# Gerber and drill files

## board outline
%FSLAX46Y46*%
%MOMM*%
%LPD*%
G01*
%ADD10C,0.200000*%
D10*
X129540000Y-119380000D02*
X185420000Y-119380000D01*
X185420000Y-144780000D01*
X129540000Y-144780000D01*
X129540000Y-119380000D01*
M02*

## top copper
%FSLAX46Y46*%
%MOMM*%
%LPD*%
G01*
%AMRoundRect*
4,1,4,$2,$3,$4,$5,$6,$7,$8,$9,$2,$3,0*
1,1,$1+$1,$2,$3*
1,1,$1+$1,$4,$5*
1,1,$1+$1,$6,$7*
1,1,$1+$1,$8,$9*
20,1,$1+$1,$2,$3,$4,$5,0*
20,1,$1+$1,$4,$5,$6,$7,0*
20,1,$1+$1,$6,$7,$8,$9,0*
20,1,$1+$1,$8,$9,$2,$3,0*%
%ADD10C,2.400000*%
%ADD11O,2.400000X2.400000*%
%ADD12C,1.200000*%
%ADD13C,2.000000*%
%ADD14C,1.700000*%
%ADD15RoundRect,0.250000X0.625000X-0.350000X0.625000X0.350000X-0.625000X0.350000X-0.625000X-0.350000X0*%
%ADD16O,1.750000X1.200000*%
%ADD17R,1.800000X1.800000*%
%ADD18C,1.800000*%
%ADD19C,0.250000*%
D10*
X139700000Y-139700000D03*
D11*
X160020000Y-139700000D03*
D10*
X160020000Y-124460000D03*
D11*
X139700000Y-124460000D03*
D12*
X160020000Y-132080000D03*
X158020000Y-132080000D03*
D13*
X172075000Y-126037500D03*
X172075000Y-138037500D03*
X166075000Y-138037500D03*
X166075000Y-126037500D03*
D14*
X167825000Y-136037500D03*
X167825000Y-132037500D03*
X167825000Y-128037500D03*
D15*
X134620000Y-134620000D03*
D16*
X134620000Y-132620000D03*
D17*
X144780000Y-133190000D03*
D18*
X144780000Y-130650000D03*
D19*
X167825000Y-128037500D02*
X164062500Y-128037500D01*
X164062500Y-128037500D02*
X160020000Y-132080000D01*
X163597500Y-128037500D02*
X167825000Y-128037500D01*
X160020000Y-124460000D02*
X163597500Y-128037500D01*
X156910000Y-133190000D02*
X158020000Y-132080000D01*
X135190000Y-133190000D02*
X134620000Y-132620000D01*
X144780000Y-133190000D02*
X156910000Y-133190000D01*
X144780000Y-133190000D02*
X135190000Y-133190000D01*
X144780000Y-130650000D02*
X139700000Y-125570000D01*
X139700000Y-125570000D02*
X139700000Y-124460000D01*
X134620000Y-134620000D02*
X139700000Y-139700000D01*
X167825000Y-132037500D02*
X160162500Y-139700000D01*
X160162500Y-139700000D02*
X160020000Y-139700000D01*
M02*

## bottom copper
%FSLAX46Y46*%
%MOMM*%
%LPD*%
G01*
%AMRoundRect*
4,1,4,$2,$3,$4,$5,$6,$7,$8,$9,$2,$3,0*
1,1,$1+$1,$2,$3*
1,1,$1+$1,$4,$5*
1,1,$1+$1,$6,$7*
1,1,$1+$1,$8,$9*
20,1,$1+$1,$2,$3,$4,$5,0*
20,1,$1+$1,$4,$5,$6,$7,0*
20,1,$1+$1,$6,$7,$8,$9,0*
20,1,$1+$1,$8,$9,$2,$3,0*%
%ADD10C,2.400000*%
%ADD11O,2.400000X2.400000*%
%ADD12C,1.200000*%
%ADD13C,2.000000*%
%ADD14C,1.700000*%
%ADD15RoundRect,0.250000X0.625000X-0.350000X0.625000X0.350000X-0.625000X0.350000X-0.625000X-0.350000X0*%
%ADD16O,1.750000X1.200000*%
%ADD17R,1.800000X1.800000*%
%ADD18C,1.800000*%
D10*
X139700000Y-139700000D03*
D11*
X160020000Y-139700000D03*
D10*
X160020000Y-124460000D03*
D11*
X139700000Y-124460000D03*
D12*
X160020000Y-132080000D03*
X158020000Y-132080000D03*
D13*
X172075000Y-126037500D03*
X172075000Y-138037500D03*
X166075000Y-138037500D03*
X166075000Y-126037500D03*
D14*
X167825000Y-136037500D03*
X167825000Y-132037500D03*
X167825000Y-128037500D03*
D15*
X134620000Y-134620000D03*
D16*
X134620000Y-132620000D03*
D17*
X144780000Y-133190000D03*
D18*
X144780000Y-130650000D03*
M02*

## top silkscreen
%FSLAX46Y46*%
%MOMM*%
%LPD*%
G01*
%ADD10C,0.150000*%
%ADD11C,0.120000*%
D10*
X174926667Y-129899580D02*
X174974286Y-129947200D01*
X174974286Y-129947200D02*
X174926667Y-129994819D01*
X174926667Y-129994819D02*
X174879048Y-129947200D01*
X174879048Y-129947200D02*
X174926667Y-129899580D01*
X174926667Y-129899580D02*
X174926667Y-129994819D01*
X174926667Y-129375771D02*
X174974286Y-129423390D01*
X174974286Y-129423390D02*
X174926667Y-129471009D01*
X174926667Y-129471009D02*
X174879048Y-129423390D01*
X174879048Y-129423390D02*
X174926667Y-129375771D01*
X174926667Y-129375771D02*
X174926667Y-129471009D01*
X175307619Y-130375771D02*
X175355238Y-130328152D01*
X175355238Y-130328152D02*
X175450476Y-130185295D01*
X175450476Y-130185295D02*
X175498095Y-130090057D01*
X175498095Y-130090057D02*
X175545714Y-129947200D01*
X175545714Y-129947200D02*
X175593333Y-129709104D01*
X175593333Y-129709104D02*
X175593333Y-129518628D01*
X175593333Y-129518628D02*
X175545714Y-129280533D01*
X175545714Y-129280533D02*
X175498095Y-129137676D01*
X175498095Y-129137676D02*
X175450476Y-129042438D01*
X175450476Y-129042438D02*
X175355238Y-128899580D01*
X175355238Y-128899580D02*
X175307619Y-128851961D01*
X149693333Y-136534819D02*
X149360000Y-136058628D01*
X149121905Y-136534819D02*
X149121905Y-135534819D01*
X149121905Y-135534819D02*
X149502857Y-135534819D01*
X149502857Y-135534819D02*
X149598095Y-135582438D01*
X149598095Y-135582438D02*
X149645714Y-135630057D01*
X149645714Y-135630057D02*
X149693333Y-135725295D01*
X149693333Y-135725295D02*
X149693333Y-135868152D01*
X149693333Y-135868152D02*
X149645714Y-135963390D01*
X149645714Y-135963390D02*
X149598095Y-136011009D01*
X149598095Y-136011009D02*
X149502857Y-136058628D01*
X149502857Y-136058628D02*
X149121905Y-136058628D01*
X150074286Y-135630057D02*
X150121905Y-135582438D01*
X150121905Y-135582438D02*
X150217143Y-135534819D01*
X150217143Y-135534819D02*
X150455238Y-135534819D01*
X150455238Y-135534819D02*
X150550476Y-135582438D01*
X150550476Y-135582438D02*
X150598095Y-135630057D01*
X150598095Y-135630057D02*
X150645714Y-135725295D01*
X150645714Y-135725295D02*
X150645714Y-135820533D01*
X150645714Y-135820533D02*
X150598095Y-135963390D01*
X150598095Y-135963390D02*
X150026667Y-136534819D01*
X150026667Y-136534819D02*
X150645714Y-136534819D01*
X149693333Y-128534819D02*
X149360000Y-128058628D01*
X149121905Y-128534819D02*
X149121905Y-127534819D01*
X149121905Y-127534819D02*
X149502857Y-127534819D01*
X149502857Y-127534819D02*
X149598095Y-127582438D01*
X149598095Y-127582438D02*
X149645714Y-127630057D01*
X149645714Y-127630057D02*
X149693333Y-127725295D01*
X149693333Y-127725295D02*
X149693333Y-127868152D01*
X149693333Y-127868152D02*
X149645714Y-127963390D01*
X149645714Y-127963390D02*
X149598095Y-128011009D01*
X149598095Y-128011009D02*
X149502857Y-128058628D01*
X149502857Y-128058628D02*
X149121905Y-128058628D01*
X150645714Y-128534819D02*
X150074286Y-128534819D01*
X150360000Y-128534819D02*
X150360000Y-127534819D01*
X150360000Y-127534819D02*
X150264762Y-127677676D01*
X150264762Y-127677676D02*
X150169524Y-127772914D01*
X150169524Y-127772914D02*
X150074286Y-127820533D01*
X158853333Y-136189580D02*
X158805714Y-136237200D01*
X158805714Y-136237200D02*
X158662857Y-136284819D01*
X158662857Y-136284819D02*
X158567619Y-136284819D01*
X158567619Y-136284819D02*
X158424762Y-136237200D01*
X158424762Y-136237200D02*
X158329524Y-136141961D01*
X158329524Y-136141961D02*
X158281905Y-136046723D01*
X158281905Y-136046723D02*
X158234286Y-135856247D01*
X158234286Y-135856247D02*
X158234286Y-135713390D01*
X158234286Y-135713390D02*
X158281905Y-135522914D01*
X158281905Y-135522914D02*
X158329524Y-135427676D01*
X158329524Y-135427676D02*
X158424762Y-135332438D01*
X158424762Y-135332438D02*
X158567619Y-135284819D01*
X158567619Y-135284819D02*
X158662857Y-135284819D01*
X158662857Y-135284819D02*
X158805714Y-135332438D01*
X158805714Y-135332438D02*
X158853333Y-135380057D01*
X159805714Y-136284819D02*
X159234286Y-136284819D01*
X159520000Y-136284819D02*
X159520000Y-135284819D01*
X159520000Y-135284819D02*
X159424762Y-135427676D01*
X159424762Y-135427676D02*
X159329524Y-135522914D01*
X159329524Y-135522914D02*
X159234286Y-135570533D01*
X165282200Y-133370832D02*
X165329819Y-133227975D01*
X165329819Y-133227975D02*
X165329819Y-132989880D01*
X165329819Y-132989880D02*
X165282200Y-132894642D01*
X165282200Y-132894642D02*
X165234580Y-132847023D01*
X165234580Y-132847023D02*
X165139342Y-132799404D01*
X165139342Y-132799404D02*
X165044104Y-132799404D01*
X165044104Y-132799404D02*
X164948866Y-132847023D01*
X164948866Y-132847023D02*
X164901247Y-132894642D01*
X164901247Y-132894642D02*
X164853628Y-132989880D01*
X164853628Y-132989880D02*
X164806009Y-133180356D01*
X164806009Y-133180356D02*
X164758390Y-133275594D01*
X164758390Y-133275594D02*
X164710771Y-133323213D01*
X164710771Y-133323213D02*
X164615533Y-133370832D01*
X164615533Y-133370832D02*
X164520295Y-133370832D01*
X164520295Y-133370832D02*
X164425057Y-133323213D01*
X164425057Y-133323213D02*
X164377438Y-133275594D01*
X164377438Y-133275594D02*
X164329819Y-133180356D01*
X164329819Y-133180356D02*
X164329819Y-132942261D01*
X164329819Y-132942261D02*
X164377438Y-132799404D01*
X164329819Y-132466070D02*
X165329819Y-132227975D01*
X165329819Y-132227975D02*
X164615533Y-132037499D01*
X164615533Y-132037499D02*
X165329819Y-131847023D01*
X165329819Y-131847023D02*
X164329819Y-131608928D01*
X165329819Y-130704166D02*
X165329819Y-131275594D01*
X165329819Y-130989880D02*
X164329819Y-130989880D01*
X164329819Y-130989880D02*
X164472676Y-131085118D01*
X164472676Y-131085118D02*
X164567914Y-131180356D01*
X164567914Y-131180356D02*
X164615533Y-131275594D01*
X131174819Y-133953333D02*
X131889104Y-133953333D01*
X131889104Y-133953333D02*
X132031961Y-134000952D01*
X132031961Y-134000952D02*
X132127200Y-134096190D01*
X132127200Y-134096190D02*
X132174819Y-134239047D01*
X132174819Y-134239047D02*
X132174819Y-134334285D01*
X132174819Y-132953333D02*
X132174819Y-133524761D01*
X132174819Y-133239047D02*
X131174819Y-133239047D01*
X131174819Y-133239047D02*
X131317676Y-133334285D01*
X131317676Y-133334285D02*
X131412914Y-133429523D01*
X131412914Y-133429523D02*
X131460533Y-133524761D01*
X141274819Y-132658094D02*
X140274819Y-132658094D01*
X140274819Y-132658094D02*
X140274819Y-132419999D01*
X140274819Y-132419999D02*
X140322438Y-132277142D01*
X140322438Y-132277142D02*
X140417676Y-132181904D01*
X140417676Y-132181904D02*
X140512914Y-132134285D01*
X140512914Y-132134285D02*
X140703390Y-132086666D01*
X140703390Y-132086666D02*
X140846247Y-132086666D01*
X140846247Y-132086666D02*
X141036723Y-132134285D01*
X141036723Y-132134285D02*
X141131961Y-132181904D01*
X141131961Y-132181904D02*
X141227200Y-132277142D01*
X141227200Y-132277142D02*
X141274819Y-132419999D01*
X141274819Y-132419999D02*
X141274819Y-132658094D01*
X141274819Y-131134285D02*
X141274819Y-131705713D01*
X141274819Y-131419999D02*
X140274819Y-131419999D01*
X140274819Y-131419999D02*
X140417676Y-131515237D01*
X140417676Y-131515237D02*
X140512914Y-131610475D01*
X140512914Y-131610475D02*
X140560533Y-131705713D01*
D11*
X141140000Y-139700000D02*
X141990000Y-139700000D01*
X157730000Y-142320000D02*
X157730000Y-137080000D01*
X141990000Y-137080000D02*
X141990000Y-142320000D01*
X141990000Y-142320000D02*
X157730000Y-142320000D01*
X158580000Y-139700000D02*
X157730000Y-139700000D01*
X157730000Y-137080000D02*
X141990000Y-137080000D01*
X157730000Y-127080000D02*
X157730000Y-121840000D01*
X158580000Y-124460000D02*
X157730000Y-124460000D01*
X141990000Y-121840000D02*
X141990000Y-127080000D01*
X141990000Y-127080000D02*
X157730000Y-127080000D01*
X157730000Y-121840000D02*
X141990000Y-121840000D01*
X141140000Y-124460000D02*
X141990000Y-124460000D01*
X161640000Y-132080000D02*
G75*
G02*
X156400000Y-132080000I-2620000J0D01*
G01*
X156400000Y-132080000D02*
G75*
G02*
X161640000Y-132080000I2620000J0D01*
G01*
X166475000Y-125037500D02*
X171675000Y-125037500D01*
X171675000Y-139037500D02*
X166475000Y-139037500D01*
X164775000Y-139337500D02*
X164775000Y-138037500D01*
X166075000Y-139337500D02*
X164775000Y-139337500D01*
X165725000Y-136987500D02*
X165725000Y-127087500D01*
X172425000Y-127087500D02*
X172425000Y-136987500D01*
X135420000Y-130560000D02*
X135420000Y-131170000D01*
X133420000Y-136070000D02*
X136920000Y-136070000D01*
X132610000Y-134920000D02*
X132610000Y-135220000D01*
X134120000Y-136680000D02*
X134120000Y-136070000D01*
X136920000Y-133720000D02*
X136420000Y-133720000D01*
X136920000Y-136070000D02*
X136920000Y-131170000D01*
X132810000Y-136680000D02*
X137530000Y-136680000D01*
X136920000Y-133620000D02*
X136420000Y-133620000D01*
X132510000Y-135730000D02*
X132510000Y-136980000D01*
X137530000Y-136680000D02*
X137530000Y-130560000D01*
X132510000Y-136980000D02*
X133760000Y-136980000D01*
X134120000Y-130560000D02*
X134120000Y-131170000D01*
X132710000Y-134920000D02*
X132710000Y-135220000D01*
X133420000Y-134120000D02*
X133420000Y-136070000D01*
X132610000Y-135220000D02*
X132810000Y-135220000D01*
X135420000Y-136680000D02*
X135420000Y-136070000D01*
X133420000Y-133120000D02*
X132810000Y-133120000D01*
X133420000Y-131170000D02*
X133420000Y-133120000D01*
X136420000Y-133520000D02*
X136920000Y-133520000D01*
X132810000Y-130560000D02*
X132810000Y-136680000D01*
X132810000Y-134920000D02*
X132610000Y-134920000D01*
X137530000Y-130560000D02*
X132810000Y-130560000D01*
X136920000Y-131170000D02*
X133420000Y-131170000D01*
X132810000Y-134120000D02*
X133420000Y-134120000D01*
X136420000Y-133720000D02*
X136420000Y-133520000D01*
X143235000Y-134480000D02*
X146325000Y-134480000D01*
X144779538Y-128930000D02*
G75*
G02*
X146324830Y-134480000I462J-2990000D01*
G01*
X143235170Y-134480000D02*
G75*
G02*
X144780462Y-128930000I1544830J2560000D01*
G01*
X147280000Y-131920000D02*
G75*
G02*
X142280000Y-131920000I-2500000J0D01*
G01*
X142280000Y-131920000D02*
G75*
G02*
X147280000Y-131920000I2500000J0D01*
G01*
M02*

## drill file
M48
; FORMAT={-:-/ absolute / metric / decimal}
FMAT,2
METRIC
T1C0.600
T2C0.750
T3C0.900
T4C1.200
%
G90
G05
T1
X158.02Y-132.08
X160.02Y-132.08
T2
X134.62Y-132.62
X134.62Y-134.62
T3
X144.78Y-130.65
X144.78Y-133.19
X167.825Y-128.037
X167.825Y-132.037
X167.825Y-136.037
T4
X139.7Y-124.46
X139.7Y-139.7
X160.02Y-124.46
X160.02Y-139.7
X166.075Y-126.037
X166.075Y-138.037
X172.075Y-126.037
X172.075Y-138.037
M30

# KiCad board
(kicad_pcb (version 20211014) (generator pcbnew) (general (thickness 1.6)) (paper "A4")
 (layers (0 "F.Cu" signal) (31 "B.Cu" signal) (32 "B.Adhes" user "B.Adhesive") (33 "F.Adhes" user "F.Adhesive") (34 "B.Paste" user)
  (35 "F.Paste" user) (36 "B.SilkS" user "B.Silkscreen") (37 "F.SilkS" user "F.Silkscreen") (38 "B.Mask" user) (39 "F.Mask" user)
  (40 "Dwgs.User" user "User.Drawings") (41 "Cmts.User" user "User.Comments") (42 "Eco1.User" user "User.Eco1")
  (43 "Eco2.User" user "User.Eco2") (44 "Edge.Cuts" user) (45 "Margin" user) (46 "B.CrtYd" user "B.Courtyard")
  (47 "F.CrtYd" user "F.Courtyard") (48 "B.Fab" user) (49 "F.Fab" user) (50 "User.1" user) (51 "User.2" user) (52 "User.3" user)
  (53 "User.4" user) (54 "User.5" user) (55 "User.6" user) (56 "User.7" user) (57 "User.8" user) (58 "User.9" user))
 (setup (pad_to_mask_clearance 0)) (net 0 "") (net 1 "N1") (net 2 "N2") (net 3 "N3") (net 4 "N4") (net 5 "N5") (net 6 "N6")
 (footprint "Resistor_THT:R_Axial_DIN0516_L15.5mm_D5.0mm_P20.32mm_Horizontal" (layer "F.Cu") (at 139.7 139.7)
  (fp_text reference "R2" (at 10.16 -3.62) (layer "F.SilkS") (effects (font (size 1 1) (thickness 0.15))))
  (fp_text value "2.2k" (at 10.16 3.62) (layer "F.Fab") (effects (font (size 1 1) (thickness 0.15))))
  (fp_line (start 1.44 0) (end 2.29 0) (layer "F.SilkS") (width 0.12))
  (fp_line (start 18.03 2.62) (end 18.03 -2.62) (layer "F.SilkS") (width 0.12))
  (fp_line (start 2.29 -2.62) (end 2.29 2.62) (layer "F.SilkS") (width 0.12))
  (fp_line (start 2.29 2.62) (end 18.03 2.62) (layer "F.SilkS") (width 0.12))
  (fp_line (start 18.88 0) (end 18.03 0) (layer "F.SilkS") (width 0.12))
  (fp_line (start 18.03 -2.62) (end 2.29 -2.62) (layer "F.SilkS") (width 0.12))
  (pad "1" thru_hole circle (at 0 0) (size 2.4 2.4) (drill 1.2) (layers *.Cu *.Mask) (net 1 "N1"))
  (pad "2" thru_hole oval (at 20.32 0) (size 2.4 2.4) (drill 1.2) (layers *.Cu *.Mask) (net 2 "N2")))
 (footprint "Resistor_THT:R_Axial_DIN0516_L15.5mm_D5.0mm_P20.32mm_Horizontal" (layer "F.Cu") (at 160.02 124.46 180)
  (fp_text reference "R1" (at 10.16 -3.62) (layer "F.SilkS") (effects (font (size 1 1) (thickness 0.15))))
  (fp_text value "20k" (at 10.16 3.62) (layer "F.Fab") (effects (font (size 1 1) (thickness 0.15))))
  (fp_line (start 2.29 -2.62) (end 2.29 2.62) (layer "F.SilkS") (width 0.12))
  (fp_line (start 1.44 0) (end 2.29 0) (layer "F.SilkS") (width 0.12))
  (fp_line (start 18.03 2.62) (end 18.03 -2.62) (layer "F.SilkS") (width 0.12))
  (fp_line (start 18.03 -2.62) (end 2.29 -2.62) (layer "F.SilkS") (width 0.12))
  (fp_line (start 2.29 2.62) (end 18.03 2.62) (layer "F.SilkS") (width 0.12))
  (fp_line (start 18.88 0) (end 18.03 0) (layer "F.SilkS") (width 0.12))
  (pad "1" thru_hole circle (at 0 0 180) (size 2.4 2.4) (drill 1.2) (layers *.Cu *.Mask) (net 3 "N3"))
  (pad "2" thru_hole oval (at 20.32 0 180) (size 2.4 2.4) (drill 1.2) (layers *.Cu *.Mask) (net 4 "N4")))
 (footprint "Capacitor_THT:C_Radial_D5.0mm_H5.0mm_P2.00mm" (layer "F.Cu") (at 160.02 132.08 180)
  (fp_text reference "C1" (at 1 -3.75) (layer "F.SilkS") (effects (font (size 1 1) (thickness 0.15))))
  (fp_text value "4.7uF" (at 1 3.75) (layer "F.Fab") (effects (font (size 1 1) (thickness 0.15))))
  (fp_circle (center 1 0) (end 3.62 0) (layer "F.SilkS") (width 0.12) (fill none))
  (pad "1" thru_hole circle (at 0 0 180) (size 1.2 1.2) (drill 0.6) (layers *.Cu *.Mask) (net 3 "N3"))
  (pad "2" thru_hole circle (at 2 0 180) (size 1.2 1.2) (drill 0.6) (layers *.Cu *.Mask) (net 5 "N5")))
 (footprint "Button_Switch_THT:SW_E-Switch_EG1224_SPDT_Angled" (layer "F.Cu") (at 167.825 136.0375 90)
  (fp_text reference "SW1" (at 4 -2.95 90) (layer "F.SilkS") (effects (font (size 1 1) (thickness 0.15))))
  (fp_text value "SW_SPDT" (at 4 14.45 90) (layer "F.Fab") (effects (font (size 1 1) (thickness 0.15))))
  (fp_line (start 11 -1.35) (end 11 3.85) (layer "F.SilkS") (width 0.12))
  (fp_line (start -3 3.85) (end -3 -1.35) (layer "F.SilkS") (width 0.12))
  (fp_line (start -3.3 -3.05) (end -2 -3.05) (layer "F.SilkS") (width 0.12))
  (fp_line (start -3.3 -1.75) (end -3.3 -3.05) (layer "F.SilkS") (width 0.12))
  (fp_line (start -0.95 -2.1) (end 8.95 -2.1) (layer "F.SilkS") (width 0.12))
  (fp_line (start 8.95 4.6) (end -0.95 4.6) (layer "F.SilkS") (width 0.12))
  (pad "" thru_hole circle (at 10 4.25 90) (size 2 2) (drill 1.2) (layers *.Cu *.Mask))
  (pad "" thru_hole circle (at -2 4.25 90) (size 2 2) (drill 1.2) (layers *.Cu *.Mask))
  (pad "" thru_hole circle (at -2 -1.75 90) (size 2 2) (drill 1.2) (layers *.Cu *.Mask))
  (pad "" thru_hole circle (at 10 -1.75 90) (size 2 2) (drill 1.2) (layers *.Cu *.Mask))
  (pad "1" thru_hole circle (at 0 0 90) (size 1.7 1.7) (drill 0.9) (layers *.Cu *.Mask) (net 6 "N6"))
  (pad "2" thru_hole circle (at 4 0 90) (size 1.7 1.7) (drill 0.9) (layers *.Cu *.Mask) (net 2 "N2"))
  (pad "3" thru_hole circle (at 8 0 90) (size 1.7 1.7) (drill 0.9) (layers *.Cu *.Mask) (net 3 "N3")))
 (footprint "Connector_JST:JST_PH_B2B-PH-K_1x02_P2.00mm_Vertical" (layer "F.Cu") (at 134.62 134.62 90)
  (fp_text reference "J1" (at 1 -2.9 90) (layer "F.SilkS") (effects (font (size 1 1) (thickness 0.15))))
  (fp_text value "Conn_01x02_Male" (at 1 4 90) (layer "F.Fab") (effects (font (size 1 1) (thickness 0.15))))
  (fp_line (start 4.06 0.8) (end 3.45 0.8) (layer "F.SilkS") (width 0.12))
  (fp_line (start -1.45 -1.2) (end -1.45 2.3) (layer "F.SilkS") (width 0.12))
  (fp_line (start -0.3 -2.01) (end -0.6 -2.01) (layer "F.SilkS") (width 0.12))
  (fp_line (start -2.06 -0.5) (end -1.45 -0.5) (layer "F.SilkS") (width 0.12))
  (fp_line (start 0.9 2.3) (end 0.9 1.8) (layer "F.SilkS") (width 0.12))
  (fp_line (start -1.45 2.3) (end 3.45 2.3) (layer "F.SilkS") (width 0.12))
  (fp_line (start -2.06 -1.81) (end -2.06 2.91) (layer "F.SilkS") (width 0.12))
  (fp_line (start 1 2.3) (end 1 1.8) (layer "F.SilkS") (width 0.12))
  (fp_line (start -1.11 -2.11) (end -2.36 -2.11) (layer "F.SilkS") (width 0.12))
  (fp_line (start -2.06 2.91) (end 4.06 2.91) (layer "F.SilkS") (width 0.12))
  (fp_line (start -2.36 -2.11) (end -2.36 -0.86) (layer "F.SilkS") (width 0.12))
  (fp_line (start 4.06 -0.5) (end 3.45 -0.5) (layer "F.SilkS") (width 0.12))
  (fp_line (start -0.3 -1.91) (end -0.6 -1.91) (layer "F.SilkS") (width 0.12))
  (fp_line (start 0.5 -1.2) (end -1.45 -1.2) (layer "F.SilkS") (width 0.12))
  (fp_line (start -0.6 -2.01) (end -0.6 -1.81) (layer "F.SilkS") (width 0.12))
  (fp_line (start -2.06 0.8) (end -1.45 0.8) (layer "F.SilkS") (width 0.12))
  (fp_line (start 1.5 -1.2) (end 1.5 -1.81) (layer "F.SilkS") (width 0.12))
  (fp_line (start 3.45 -1.2) (end 1.5 -1.2) (layer "F.SilkS") (width 0.12))
  (fp_line (start 1.1 1.8) (end 1.1 2.3) (layer "F.SilkS") (width 0.12))
  (fp_line (start 4.06 -1.81) (end -2.06 -1.81) (layer "F.SilkS") (width 0.12))
  (fp_line (start -0.3 -1.81) (end -0.3 -2.01) (layer "F.SilkS") (width 0.12))
  (fp_line (start 4.06 2.91) (end 4.06 -1.81) (layer "F.SilkS") (width 0.12))
  (fp_line (start 3.45 2.3) (end 3.45 -1.2) (layer "F.SilkS") (width 0.12))
  (fp_line (start 0.5 -1.81) (end 0.5 -1.2) (layer "F.SilkS") (width 0.12))
  (fp_line (start 0.9 1.8) (end 1.1 1.8) (layer "F.SilkS") (width 0.12))
  (pad "1" thru_hole roundrect (at 0 0 90) (size 1.2 1.75) (drill 0.75) (layers *.Cu *.Mask) (roundrect_rratio 0.208333) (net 1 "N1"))
  (pad "2" thru_hole oval (at 2 0 90) (size 1.2 1.75) (drill 0.75) (layers *.Cu *.Mask) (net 5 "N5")))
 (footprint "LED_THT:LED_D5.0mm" (layer "F.Cu") (at 144.78 133.19 90)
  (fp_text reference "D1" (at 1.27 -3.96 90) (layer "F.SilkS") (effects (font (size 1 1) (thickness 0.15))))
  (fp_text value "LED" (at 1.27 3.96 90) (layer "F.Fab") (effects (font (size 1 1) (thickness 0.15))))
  (fp_line (start -1.29 -1.545) (end -1.29 1.545) (layer "F.SilkS") (width 0.12))
  (fp_arc (start 4.26 -0.000462) (mid 2.072002 2.880433) (end -1.29 1.54483) (layer "F.SilkS") (width 0.12))
  (fp_arc (start -1.29 -1.54483) (mid 2.072002 -2.880433) (end 4.26 0.000462) (layer "F.SilkS") (width 0.12))
  (fp_circle (center 1.27 0) (end 3.77 0) (layer "F.SilkS") (width 0.12) (fill none))
  (pad "1" thru_hole rect (at 0 0 90) (size 1.8 1.8) (drill 0.9) (layers *.Cu *.Mask) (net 5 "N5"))
  (pad "2" thru_hole circle (at 2.54 0 90) (size 1.8 1.8) (drill 0.9) (layers *.Cu *.Mask) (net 4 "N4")))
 (gr_rect (start 129.54 119.38) (end 185.42 144.78) (layer "Edge.Cuts") (width 0.2) (fill none))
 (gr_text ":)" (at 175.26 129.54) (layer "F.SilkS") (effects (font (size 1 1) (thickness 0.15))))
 (segment (start 167.825 128.0375) (end 164.0625 128.0375) (width 0.25) (layer "F.Cu") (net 3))
 (segment (start 164.0625 128.0375) (end 160.02 132.08) (width 0.25) (layer "F.Cu") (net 3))
 (segment (start 163.5975 128.0375) (end 167.825 128.0375) (width 0.25) (layer "F.Cu") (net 3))
 (segment (start 160.02 124.46) (end 163.5975 128.0375) (width 0.25) (layer "F.Cu") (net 3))
 (segment (start 156.91 133.19) (end 158.02 132.08) (width 0.25) (layer "F.Cu") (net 5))
 (segment (start 135.19 133.19) (end 134.62 132.62) (width 0.25) (layer "F.Cu") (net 5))
 (segment (start 144.78 133.19) (end 156.91 133.19) (width 0.25) (layer "F.Cu") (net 5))
 (segment (start 144.78 133.19) (end 135.19 133.19) (width 0.25) (layer "F.Cu") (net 5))
 (segment (start 144.78 130.65) (end 139.7 125.57) (width 0.25) (layer "F.Cu") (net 4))
 (segment (start 139.7 125.57) (end 139.7 124.46) (width 0.25) (layer "F.Cu") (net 4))
 (segment (start 134.62 134.62) (end 139.7 139.7) (width 0.25) (layer "F.Cu") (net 1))
 (segment (start 167.825 132.0375) (end 160.1625 139.7) (width 0.25) (layer "F.Cu") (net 2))
 (segment (start 160.1625 139.7) (end 160.02 139.7) (width 0.25) (layer "F.Cu") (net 2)))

